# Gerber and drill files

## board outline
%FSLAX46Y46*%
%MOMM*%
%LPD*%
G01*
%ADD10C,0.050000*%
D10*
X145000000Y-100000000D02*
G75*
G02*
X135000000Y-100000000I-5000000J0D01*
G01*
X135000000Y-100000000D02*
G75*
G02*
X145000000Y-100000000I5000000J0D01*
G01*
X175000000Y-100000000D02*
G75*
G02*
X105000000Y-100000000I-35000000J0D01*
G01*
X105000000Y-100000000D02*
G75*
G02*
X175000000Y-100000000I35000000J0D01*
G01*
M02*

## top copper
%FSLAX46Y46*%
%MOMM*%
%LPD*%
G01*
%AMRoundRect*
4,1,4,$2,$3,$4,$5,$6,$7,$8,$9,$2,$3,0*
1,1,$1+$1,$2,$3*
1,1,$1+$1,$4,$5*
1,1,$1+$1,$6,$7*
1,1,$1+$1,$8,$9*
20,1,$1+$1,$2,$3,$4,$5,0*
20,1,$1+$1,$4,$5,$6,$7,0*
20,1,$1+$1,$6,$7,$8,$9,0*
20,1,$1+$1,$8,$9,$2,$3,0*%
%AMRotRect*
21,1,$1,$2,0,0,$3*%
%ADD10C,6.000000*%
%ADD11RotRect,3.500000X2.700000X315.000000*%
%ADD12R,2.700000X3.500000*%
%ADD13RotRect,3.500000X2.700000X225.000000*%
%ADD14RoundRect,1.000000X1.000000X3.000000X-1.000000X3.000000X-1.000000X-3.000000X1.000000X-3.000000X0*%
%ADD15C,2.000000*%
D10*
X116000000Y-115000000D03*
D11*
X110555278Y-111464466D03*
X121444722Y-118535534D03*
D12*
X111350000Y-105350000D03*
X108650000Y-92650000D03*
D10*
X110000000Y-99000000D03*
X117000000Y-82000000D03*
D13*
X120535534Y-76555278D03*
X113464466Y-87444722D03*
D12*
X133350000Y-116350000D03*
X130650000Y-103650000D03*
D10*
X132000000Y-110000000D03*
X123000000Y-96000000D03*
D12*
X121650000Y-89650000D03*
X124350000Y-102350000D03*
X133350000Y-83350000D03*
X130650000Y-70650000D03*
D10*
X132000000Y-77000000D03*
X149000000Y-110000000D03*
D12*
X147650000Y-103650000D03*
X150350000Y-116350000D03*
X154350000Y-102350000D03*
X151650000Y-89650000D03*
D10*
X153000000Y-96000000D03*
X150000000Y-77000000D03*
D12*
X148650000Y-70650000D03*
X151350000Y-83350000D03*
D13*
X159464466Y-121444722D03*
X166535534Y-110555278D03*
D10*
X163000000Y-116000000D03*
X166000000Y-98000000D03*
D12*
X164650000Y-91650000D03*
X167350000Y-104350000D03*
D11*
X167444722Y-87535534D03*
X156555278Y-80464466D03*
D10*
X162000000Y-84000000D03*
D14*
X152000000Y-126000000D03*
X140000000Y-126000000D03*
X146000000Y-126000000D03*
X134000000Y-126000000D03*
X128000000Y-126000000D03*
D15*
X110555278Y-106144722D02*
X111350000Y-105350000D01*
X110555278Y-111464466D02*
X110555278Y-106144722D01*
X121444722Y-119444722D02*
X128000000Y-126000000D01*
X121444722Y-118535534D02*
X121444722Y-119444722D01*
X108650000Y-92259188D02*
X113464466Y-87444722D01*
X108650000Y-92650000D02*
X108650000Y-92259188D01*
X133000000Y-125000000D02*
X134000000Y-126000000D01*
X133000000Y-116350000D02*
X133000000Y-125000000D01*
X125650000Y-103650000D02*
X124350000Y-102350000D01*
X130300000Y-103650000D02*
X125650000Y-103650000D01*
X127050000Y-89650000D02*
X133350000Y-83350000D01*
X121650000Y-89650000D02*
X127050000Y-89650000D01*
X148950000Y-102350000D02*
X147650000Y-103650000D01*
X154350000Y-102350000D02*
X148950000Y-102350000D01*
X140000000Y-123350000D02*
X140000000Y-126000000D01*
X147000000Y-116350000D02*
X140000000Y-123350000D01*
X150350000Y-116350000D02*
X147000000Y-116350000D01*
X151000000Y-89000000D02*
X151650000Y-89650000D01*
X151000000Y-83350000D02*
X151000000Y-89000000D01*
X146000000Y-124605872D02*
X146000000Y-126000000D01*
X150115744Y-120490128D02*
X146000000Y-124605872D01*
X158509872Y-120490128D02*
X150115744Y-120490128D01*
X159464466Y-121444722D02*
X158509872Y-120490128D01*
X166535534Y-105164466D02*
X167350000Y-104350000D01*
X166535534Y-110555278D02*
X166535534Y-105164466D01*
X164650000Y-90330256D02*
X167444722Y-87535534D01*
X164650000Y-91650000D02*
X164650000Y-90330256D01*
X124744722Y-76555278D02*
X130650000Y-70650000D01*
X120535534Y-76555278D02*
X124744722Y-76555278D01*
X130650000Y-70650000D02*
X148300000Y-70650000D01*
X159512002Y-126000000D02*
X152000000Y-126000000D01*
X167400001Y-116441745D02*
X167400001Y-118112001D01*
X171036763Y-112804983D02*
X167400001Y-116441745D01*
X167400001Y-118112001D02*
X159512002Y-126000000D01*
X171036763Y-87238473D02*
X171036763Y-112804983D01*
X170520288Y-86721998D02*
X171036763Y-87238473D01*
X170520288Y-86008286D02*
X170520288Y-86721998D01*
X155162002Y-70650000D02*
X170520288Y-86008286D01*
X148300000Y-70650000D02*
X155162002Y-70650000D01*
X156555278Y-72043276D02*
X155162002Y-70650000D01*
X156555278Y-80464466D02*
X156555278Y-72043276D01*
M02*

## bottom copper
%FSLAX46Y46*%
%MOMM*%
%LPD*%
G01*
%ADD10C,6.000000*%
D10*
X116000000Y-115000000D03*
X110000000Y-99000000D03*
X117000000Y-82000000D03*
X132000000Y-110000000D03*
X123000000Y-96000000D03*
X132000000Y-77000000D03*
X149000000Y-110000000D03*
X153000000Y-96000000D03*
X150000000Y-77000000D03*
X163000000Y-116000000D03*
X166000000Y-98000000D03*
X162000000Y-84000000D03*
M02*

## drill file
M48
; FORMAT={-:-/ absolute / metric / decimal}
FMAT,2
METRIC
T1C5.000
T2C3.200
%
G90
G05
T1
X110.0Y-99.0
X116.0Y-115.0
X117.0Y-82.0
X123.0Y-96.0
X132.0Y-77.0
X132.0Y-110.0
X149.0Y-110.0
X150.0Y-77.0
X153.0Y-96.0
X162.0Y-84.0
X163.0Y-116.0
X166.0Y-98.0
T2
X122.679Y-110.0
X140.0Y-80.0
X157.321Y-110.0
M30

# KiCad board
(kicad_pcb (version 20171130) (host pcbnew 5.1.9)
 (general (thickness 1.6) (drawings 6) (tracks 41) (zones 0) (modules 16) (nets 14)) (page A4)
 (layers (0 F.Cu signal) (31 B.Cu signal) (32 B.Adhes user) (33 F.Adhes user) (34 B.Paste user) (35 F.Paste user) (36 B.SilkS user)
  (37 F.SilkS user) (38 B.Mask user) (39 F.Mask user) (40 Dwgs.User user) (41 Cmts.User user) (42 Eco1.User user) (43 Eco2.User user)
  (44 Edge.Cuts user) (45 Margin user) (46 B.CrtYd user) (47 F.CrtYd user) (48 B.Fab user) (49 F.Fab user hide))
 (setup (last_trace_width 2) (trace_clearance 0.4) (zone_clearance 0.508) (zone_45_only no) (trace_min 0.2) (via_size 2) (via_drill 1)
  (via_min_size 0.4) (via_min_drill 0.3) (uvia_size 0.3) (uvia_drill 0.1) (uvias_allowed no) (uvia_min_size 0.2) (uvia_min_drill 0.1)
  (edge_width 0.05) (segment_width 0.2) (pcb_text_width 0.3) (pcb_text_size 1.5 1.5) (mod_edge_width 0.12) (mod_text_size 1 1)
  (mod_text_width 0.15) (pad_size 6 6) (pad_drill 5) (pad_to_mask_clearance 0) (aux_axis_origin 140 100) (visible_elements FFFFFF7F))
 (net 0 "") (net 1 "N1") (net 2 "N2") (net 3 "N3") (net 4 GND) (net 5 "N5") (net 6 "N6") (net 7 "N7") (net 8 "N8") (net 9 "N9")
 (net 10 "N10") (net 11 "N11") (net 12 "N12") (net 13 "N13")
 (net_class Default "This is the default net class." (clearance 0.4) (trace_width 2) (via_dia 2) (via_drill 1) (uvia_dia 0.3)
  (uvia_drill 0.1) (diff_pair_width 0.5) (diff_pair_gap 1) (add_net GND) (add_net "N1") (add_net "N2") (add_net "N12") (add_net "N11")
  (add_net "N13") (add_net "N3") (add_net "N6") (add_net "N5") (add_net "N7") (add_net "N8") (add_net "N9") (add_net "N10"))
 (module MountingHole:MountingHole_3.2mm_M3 (layer F.Cu) (at 157.320508 110 240)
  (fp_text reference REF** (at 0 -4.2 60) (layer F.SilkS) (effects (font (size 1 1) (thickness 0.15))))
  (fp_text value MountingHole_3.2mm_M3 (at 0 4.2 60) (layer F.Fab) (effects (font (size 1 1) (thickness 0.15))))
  (pad 1 np_thru_hole circle (at 0 0 240) (size 3.2 3.2) (drill 3.2) (layers *.Cu *.Mask)))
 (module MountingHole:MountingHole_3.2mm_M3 (layer F.Cu) (at 122.679492 110 120)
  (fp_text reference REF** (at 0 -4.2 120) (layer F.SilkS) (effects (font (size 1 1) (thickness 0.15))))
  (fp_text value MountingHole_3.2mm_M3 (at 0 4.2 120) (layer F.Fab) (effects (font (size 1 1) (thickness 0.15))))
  (pad 1 np_thru_hole circle (at 0 0 120) (size 3.2 3.2) (drill 3.2) (layers *.Cu *.Mask)))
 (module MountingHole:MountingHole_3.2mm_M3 (layer F.Cu) (at 140 80)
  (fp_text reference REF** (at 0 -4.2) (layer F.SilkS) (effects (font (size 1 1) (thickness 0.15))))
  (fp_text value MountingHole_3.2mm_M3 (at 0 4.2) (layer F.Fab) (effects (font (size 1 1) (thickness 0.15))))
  (pad 1 np_thru_hole circle (at 0 0) (size 3.2 3.2) (drill 3.2) (layers *.Cu *.Mask)))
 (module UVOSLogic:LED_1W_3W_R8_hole (layer F.Cu) (at 116 115 315)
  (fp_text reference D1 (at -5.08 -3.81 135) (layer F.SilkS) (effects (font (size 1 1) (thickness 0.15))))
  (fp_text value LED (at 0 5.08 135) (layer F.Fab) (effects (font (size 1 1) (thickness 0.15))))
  (pad 3 thru_hole circle (at 0 0 315) (size 6 6) (drill 5) (layers *.Cu *.Mask))
  (pad 1 smd rect (at -6.35 1.35 315) (size 3.5 2.7) (layers F.Cu F.Paste F.Mask) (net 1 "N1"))
  (pad 2 smd rect (at 6.35 -1.35 315) (size 3.5 2.7) (layers F.Cu F.Paste F.Mask) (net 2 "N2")))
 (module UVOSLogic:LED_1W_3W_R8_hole (layer F.Cu) (at 110 99 270)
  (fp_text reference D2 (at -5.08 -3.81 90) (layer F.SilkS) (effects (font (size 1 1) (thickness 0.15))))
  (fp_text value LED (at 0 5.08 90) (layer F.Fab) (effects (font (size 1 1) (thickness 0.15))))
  (pad 2 smd rect (at 6.35 -1.35 270) (size 3.5 2.7) (layers F.Cu F.Paste F.Mask) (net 1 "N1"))
  (pad 1 smd rect (at -6.35 1.35 270) (size 3.5 2.7) (layers F.Cu F.Paste F.Mask) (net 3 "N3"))
  (pad 3 thru_hole circle (at 0 0 270) (size 6 6) (drill 5) (layers *.Cu *.Mask)))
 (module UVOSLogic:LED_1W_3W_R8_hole (layer F.Cu) (at 117 82 225)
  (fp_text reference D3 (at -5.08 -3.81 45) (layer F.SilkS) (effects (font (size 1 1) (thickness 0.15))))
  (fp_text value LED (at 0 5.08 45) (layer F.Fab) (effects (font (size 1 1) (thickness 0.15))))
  (pad 3 thru_hole circle (at 0 0 225) (size 6 6) (drill 5) (layers *.Cu *.Mask))
  (pad 1 smd rect (at -6.35 1.35 225) (size 3.5 2.7) (layers F.Cu F.Paste F.Mask) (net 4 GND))
  (pad 2 smd rect (at 6.35 -1.35 225) (size 3.5 2.7) (layers F.Cu F.Paste F.Mask) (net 3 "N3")))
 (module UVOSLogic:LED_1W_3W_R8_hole (layer F.Cu) (at 132 110 270)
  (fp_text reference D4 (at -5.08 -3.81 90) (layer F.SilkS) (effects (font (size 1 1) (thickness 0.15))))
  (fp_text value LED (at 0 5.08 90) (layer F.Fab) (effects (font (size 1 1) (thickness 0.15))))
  (pad 2 smd rect (at 6.35 -1.35 270) (size 3.5 2.7) (layers F.Cu F.Paste F.Mask) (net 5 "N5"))
  (pad 1 smd rect (at -6.35 1.35 270) (size 3.5 2.7) (layers F.Cu F.Paste F.Mask) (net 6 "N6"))
  (pad 3 thru_hole circle (at 0 0 270) (size 6 6) (drill 5) (layers *.Cu *.Mask)))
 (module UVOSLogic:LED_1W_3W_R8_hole (layer F.Cu) (at 123 96 270)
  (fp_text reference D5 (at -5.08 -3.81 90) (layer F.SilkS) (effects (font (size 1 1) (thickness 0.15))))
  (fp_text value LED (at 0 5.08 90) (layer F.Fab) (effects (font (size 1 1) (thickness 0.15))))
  (pad 3 thru_hole circle (at 0 0 270) (size 6 6) (drill 5) (layers *.Cu *.Mask))
  (pad 1 smd rect (at -6.35 1.35 270) (size 3.5 2.7) (layers F.Cu F.Paste F.Mask) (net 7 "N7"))
  (pad 2 smd rect (at 6.35 -1.35 270) (size 3.5 2.7) (layers F.Cu F.Paste F.Mask) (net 6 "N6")))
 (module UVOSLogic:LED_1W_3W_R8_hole (layer F.Cu) (at 132 77 270)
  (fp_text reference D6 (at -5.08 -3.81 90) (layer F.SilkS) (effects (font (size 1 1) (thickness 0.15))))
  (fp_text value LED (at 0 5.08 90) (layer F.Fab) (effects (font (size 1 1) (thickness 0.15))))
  (pad 2 smd rect (at 6.35 -1.35 270) (size 3.5 2.7) (layers F.Cu F.Paste F.Mask) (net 7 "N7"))
  (pad 1 smd rect (at -6.35 1.35 270) (size 3.5 2.7) (layers F.Cu F.Paste F.Mask) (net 4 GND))
  (pad 3 thru_hole circle (at 0 0 270) (size 6 6) (drill 5) (layers *.Cu *.Mask)))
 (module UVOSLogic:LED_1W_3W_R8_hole (layer F.Cu) (at 149 110 270)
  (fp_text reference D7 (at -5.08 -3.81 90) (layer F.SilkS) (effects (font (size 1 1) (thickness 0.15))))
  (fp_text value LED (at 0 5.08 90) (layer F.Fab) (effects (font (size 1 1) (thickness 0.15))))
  (pad 3 thru_hole circle (at 0 0 270) (size 6 6) (drill 5) (layers *.Cu *.Mask))
  (pad 1 smd rect (at -6.35 1.35 270) (size 3.5 2.7) (layers F.Cu F.Paste F.Mask) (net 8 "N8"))
  (pad 2 smd rect (at 6.35 -1.35 270) (size 3.5 2.7) (layers F.Cu F.Paste F.Mask) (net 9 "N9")))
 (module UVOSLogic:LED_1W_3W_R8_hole (layer F.Cu) (at 153 96 270)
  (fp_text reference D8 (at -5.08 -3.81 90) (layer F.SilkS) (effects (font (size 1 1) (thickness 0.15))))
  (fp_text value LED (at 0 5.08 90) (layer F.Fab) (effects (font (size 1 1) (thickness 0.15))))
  (pad 2 smd rect (at 6.35 -1.35 270) (size 3.5 2.7) (layers F.Cu F.Paste F.Mask) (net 8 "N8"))
  (pad 1 smd rect (at -6.35 1.35 270) (size 3.5 2.7) (layers F.Cu F.Paste F.Mask) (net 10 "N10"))
  (pad 3 thru_hole circle (at 0 0 270) (size 6 6) (drill 5) (layers *.Cu *.Mask)))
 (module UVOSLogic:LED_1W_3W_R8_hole (layer F.Cu) (at 150 77 270)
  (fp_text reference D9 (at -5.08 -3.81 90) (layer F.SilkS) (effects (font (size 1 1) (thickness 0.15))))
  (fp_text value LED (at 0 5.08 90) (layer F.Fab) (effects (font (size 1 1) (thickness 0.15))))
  (pad 3 thru_hole circle (at 0 0 270) (size 6 6) (drill 5) (layers *.Cu *.Mask))
  (pad 1 smd rect (at -6.35 1.35 270) (size 3.5 2.7) (layers F.Cu F.Paste F.Mask) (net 4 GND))
  (pad 2 smd rect (at 6.35 -1.35 270) (size 3.5 2.7) (layers F.Cu F.Paste F.Mask) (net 10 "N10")))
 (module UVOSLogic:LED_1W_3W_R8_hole (layer F.Cu) (at 163 116 225)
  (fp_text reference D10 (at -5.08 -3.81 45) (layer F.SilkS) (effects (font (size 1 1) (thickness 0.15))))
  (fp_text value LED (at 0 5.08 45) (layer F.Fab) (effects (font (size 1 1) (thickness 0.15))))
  (pad 2 smd rect (at 6.35 -1.35 225) (size 3.5 2.7) (layers F.Cu F.Paste F.Mask) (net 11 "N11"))
  (pad 1 smd rect (at -6.35 1.35 225) (size 3.5 2.7) (layers F.Cu F.Paste F.Mask) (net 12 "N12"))
  (pad 3 thru_hole circle (at 0 0 225) (size 6 6) (drill 5) (layers *.Cu *.Mask)))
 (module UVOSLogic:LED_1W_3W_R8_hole (layer F.Cu) (at 166 98 270)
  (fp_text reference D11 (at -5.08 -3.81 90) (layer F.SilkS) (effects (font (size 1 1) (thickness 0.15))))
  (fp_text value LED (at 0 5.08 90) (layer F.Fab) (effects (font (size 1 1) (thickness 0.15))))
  (pad 3 thru_hole circle (at 0 0 270) (size 6 6) (drill 5) (layers *.Cu *.Mask))
  (pad 1 smd rect (at -6.35 1.35 270) (size 3.5 2.7) (layers F.Cu F.Paste F.Mask) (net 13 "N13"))
  (pad 2 smd rect (at 6.35 -1.35 270) (size 3.5 2.7) (layers F.Cu F.Paste F.Mask) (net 12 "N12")))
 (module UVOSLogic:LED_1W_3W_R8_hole (layer F.Cu) (at 162 84 315)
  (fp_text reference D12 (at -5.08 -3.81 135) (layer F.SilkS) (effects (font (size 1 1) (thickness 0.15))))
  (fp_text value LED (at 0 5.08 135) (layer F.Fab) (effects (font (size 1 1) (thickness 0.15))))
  (pad 2 smd rect (at 6.35 -1.35 315) (size 3.5 2.7) (layers F.Cu F.Paste F.Mask) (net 13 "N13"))
  (pad 1 smd rect (at -6.35 1.35 315) (size 3.5 2.7) (layers F.Cu F.Paste F.Mask) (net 4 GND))
  (pad 3 thru_hole circle (at 0 0 315) (size 6 6) (drill 5) (layers *.Cu *.Mask)))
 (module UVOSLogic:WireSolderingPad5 (layer F.Cu) (at 140 126 180)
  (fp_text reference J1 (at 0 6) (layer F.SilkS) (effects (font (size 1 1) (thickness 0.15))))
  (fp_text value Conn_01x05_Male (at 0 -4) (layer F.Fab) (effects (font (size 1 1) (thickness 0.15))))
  (pad 1 smd roundrect (at -12 0 180) (size 4 8) (layers F.Cu F.Paste F.Mask) (roundrect_rratio 0.25) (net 4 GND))
  (pad 3 smd roundrect (at 0 0 180) (size 4 8) (layers F.Cu F.Paste F.Mask) (roundrect_rratio 0.25) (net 9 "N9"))
  (pad 2 smd roundrect (at -6 0 180) (size 4 8) (layers F.Cu F.Paste F.Mask) (roundrect_rratio 0.25) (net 11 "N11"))
  (pad 4 smd roundrect (at 6 0 180) (size 4 8) (layers F.Cu F.Paste F.Mask) (roundrect_rratio 0.25) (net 5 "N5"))
  (pad 5 smd roundrect (at 12 0 180) (size 4 8) (layers F.Cu F.Paste F.Mask) (roundrect_rratio 0.25) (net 2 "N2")))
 (gr_circle (center 140 100) (end 145 100) (layer Edge.Cuts) (width 0.05))
 (gr_circle (center 140 100) (end 175 100) (layer Edge.Cuts) (width 0.05))
 (segment (start 110.555278 106.144722) (end 111.35 105.35) (width 2) (layer F.Cu) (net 1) (status 30))
 (segment (start 110.555278 111.464466) (end 110.555278 106.144722) (width 2) (layer F.Cu) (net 1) (status 30))
 (segment (start 121.444722 119.444722) (end 128 126) (width 2) (layer F.Cu) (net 2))
 (segment (start 121.444722 118.535534) (end 121.444722 119.444722) (width 2) (layer F.Cu) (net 2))
 (segment (start 108.65 92.259188) (end 113.464466 87.444722) (width 2) (layer F.Cu) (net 3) (status 30))
 (segment (start 108.65 92.65) (end 108.65 92.259188) (width 2) (layer F.Cu) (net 3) (status 30))
 (segment (start 133 125) (end 134 126) (width 2) (layer F.Cu) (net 5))
 (segment (start 133 116.35) (end 133 125) (width 2) (layer F.Cu) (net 5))
 (segment (start 125.65 103.65) (end 124.35 102.35) (width 2) (layer F.Cu) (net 6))
 (segment (start 130.3 103.65) (end 125.65 103.65) (width 2) (layer F.Cu) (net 6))
 (segment (start 127.05 89.65) (end 133.35 83.35) (width 2) (layer F.Cu) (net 7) (status 20))
 (segment (start 121.65 89.65) (end 127.05 89.65) (width 2) (layer F.Cu) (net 7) (status 10))
 (segment (start 148.95 102.35) (end 147.65 103.65) (width 2) (layer F.Cu) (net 8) (status 30))
 (segment (start 154.35 102.35) (end 148.95 102.35) (width 2) (layer F.Cu) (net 8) (status 30))
 (segment (start 140 123.35) (end 140 126) (width 2) (layer F.Cu) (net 9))
 (segment (start 147 116.35) (end 140 123.35) (width 2) (layer F.Cu) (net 9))
 (segment (start 150.35 116.35) (end 147 116.35) (width 2) (layer F.Cu) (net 9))
 (segment (start 151 89) (end 151.65 89.65) (width 2) (layer F.Cu) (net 10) (status 30))
 (segment (start 151 83.35) (end 151 89) (width 2) (layer F.Cu) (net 10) (status 30))
 (segment (start 146 124.605872) (end 146 126) (width 2) (layer F.Cu) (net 11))
 (segment (start 150.115744 120.490128) (end 146 124.605872) (width 2) (layer F.Cu) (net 11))
 (segment (start 158.509872 120.490128) (end 150.115744 120.490128) (width 2) (layer F.Cu) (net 11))
 (segment (start 159.464466 121.444722) (end 158.509872 120.490128) (width 2) (layer F.Cu) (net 11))
 (segment (start 166.535534 105.164466) (end 167.35 104.35) (width 2) (layer F.Cu) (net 12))
 (segment (start 166.535534 110.555278) (end 166.535534 105.164466) (width 2) (layer F.Cu) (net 12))
 (segment (start 164.65 90.330256) (end 167.444722 87.535534) (width 2) (layer F.Cu) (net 13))
 (segment (start 164.65 91.65) (end 164.65 90.330256) (width 2) (layer F.Cu) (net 13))
 (segment (start 124.744722 76.555278) (end 130.65 70.65) (width 2) (layer F.Cu) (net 4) (status 20))
 (segment (start 120.535534 76.555278) (end 124.744722 76.555278) (width 2) (layer F.Cu) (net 4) (status 10))
 (segment (start 130.65 70.65) (end 148.3 70.65) (width 2) (layer F.Cu) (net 4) (status 30))
 (segment (start 159.512002 126) (end 152 126) (width 2) (layer F.Cu) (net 4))
 (segment (start 167.400001 116.441745) (end 167.400001 118.112001) (width 2) (layer F.Cu) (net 4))
 (segment (start 171.036763 112.804983) (end 167.400001 116.441745) (width 2) (layer F.Cu) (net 4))
 (segment (start 167.400001 118.112001) (end 159.512002 126) (width 2) (layer F.Cu) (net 4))
 (segment (start 171.036763 87.238473) (end 171.036763 112.804983) (width 2) (layer F.Cu) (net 4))
 (segment (start 170.520288 86.721998) (end 171.036763 87.238473) (width 2) (layer F.Cu) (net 4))
 (segment (start 170.520288 86.008286) (end 170.520288 86.721998) (width 2) (layer F.Cu) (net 4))
 (segment (start 155.162002 70.65) (end 170.520288 86.008286) (width 2) (layer F.Cu) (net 4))
 (segment (start 148.3 70.65) (end 155.162002 70.65) (width 2) (layer F.Cu) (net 4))
 (segment (start 156.555278 72.043276) (end 155.162002 70.65) (width 2) (layer F.Cu) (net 4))
 (segment (start 156.555278 80.464466) (end 156.555278 72.043276) (width 2) (layer F.Cu) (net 4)))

